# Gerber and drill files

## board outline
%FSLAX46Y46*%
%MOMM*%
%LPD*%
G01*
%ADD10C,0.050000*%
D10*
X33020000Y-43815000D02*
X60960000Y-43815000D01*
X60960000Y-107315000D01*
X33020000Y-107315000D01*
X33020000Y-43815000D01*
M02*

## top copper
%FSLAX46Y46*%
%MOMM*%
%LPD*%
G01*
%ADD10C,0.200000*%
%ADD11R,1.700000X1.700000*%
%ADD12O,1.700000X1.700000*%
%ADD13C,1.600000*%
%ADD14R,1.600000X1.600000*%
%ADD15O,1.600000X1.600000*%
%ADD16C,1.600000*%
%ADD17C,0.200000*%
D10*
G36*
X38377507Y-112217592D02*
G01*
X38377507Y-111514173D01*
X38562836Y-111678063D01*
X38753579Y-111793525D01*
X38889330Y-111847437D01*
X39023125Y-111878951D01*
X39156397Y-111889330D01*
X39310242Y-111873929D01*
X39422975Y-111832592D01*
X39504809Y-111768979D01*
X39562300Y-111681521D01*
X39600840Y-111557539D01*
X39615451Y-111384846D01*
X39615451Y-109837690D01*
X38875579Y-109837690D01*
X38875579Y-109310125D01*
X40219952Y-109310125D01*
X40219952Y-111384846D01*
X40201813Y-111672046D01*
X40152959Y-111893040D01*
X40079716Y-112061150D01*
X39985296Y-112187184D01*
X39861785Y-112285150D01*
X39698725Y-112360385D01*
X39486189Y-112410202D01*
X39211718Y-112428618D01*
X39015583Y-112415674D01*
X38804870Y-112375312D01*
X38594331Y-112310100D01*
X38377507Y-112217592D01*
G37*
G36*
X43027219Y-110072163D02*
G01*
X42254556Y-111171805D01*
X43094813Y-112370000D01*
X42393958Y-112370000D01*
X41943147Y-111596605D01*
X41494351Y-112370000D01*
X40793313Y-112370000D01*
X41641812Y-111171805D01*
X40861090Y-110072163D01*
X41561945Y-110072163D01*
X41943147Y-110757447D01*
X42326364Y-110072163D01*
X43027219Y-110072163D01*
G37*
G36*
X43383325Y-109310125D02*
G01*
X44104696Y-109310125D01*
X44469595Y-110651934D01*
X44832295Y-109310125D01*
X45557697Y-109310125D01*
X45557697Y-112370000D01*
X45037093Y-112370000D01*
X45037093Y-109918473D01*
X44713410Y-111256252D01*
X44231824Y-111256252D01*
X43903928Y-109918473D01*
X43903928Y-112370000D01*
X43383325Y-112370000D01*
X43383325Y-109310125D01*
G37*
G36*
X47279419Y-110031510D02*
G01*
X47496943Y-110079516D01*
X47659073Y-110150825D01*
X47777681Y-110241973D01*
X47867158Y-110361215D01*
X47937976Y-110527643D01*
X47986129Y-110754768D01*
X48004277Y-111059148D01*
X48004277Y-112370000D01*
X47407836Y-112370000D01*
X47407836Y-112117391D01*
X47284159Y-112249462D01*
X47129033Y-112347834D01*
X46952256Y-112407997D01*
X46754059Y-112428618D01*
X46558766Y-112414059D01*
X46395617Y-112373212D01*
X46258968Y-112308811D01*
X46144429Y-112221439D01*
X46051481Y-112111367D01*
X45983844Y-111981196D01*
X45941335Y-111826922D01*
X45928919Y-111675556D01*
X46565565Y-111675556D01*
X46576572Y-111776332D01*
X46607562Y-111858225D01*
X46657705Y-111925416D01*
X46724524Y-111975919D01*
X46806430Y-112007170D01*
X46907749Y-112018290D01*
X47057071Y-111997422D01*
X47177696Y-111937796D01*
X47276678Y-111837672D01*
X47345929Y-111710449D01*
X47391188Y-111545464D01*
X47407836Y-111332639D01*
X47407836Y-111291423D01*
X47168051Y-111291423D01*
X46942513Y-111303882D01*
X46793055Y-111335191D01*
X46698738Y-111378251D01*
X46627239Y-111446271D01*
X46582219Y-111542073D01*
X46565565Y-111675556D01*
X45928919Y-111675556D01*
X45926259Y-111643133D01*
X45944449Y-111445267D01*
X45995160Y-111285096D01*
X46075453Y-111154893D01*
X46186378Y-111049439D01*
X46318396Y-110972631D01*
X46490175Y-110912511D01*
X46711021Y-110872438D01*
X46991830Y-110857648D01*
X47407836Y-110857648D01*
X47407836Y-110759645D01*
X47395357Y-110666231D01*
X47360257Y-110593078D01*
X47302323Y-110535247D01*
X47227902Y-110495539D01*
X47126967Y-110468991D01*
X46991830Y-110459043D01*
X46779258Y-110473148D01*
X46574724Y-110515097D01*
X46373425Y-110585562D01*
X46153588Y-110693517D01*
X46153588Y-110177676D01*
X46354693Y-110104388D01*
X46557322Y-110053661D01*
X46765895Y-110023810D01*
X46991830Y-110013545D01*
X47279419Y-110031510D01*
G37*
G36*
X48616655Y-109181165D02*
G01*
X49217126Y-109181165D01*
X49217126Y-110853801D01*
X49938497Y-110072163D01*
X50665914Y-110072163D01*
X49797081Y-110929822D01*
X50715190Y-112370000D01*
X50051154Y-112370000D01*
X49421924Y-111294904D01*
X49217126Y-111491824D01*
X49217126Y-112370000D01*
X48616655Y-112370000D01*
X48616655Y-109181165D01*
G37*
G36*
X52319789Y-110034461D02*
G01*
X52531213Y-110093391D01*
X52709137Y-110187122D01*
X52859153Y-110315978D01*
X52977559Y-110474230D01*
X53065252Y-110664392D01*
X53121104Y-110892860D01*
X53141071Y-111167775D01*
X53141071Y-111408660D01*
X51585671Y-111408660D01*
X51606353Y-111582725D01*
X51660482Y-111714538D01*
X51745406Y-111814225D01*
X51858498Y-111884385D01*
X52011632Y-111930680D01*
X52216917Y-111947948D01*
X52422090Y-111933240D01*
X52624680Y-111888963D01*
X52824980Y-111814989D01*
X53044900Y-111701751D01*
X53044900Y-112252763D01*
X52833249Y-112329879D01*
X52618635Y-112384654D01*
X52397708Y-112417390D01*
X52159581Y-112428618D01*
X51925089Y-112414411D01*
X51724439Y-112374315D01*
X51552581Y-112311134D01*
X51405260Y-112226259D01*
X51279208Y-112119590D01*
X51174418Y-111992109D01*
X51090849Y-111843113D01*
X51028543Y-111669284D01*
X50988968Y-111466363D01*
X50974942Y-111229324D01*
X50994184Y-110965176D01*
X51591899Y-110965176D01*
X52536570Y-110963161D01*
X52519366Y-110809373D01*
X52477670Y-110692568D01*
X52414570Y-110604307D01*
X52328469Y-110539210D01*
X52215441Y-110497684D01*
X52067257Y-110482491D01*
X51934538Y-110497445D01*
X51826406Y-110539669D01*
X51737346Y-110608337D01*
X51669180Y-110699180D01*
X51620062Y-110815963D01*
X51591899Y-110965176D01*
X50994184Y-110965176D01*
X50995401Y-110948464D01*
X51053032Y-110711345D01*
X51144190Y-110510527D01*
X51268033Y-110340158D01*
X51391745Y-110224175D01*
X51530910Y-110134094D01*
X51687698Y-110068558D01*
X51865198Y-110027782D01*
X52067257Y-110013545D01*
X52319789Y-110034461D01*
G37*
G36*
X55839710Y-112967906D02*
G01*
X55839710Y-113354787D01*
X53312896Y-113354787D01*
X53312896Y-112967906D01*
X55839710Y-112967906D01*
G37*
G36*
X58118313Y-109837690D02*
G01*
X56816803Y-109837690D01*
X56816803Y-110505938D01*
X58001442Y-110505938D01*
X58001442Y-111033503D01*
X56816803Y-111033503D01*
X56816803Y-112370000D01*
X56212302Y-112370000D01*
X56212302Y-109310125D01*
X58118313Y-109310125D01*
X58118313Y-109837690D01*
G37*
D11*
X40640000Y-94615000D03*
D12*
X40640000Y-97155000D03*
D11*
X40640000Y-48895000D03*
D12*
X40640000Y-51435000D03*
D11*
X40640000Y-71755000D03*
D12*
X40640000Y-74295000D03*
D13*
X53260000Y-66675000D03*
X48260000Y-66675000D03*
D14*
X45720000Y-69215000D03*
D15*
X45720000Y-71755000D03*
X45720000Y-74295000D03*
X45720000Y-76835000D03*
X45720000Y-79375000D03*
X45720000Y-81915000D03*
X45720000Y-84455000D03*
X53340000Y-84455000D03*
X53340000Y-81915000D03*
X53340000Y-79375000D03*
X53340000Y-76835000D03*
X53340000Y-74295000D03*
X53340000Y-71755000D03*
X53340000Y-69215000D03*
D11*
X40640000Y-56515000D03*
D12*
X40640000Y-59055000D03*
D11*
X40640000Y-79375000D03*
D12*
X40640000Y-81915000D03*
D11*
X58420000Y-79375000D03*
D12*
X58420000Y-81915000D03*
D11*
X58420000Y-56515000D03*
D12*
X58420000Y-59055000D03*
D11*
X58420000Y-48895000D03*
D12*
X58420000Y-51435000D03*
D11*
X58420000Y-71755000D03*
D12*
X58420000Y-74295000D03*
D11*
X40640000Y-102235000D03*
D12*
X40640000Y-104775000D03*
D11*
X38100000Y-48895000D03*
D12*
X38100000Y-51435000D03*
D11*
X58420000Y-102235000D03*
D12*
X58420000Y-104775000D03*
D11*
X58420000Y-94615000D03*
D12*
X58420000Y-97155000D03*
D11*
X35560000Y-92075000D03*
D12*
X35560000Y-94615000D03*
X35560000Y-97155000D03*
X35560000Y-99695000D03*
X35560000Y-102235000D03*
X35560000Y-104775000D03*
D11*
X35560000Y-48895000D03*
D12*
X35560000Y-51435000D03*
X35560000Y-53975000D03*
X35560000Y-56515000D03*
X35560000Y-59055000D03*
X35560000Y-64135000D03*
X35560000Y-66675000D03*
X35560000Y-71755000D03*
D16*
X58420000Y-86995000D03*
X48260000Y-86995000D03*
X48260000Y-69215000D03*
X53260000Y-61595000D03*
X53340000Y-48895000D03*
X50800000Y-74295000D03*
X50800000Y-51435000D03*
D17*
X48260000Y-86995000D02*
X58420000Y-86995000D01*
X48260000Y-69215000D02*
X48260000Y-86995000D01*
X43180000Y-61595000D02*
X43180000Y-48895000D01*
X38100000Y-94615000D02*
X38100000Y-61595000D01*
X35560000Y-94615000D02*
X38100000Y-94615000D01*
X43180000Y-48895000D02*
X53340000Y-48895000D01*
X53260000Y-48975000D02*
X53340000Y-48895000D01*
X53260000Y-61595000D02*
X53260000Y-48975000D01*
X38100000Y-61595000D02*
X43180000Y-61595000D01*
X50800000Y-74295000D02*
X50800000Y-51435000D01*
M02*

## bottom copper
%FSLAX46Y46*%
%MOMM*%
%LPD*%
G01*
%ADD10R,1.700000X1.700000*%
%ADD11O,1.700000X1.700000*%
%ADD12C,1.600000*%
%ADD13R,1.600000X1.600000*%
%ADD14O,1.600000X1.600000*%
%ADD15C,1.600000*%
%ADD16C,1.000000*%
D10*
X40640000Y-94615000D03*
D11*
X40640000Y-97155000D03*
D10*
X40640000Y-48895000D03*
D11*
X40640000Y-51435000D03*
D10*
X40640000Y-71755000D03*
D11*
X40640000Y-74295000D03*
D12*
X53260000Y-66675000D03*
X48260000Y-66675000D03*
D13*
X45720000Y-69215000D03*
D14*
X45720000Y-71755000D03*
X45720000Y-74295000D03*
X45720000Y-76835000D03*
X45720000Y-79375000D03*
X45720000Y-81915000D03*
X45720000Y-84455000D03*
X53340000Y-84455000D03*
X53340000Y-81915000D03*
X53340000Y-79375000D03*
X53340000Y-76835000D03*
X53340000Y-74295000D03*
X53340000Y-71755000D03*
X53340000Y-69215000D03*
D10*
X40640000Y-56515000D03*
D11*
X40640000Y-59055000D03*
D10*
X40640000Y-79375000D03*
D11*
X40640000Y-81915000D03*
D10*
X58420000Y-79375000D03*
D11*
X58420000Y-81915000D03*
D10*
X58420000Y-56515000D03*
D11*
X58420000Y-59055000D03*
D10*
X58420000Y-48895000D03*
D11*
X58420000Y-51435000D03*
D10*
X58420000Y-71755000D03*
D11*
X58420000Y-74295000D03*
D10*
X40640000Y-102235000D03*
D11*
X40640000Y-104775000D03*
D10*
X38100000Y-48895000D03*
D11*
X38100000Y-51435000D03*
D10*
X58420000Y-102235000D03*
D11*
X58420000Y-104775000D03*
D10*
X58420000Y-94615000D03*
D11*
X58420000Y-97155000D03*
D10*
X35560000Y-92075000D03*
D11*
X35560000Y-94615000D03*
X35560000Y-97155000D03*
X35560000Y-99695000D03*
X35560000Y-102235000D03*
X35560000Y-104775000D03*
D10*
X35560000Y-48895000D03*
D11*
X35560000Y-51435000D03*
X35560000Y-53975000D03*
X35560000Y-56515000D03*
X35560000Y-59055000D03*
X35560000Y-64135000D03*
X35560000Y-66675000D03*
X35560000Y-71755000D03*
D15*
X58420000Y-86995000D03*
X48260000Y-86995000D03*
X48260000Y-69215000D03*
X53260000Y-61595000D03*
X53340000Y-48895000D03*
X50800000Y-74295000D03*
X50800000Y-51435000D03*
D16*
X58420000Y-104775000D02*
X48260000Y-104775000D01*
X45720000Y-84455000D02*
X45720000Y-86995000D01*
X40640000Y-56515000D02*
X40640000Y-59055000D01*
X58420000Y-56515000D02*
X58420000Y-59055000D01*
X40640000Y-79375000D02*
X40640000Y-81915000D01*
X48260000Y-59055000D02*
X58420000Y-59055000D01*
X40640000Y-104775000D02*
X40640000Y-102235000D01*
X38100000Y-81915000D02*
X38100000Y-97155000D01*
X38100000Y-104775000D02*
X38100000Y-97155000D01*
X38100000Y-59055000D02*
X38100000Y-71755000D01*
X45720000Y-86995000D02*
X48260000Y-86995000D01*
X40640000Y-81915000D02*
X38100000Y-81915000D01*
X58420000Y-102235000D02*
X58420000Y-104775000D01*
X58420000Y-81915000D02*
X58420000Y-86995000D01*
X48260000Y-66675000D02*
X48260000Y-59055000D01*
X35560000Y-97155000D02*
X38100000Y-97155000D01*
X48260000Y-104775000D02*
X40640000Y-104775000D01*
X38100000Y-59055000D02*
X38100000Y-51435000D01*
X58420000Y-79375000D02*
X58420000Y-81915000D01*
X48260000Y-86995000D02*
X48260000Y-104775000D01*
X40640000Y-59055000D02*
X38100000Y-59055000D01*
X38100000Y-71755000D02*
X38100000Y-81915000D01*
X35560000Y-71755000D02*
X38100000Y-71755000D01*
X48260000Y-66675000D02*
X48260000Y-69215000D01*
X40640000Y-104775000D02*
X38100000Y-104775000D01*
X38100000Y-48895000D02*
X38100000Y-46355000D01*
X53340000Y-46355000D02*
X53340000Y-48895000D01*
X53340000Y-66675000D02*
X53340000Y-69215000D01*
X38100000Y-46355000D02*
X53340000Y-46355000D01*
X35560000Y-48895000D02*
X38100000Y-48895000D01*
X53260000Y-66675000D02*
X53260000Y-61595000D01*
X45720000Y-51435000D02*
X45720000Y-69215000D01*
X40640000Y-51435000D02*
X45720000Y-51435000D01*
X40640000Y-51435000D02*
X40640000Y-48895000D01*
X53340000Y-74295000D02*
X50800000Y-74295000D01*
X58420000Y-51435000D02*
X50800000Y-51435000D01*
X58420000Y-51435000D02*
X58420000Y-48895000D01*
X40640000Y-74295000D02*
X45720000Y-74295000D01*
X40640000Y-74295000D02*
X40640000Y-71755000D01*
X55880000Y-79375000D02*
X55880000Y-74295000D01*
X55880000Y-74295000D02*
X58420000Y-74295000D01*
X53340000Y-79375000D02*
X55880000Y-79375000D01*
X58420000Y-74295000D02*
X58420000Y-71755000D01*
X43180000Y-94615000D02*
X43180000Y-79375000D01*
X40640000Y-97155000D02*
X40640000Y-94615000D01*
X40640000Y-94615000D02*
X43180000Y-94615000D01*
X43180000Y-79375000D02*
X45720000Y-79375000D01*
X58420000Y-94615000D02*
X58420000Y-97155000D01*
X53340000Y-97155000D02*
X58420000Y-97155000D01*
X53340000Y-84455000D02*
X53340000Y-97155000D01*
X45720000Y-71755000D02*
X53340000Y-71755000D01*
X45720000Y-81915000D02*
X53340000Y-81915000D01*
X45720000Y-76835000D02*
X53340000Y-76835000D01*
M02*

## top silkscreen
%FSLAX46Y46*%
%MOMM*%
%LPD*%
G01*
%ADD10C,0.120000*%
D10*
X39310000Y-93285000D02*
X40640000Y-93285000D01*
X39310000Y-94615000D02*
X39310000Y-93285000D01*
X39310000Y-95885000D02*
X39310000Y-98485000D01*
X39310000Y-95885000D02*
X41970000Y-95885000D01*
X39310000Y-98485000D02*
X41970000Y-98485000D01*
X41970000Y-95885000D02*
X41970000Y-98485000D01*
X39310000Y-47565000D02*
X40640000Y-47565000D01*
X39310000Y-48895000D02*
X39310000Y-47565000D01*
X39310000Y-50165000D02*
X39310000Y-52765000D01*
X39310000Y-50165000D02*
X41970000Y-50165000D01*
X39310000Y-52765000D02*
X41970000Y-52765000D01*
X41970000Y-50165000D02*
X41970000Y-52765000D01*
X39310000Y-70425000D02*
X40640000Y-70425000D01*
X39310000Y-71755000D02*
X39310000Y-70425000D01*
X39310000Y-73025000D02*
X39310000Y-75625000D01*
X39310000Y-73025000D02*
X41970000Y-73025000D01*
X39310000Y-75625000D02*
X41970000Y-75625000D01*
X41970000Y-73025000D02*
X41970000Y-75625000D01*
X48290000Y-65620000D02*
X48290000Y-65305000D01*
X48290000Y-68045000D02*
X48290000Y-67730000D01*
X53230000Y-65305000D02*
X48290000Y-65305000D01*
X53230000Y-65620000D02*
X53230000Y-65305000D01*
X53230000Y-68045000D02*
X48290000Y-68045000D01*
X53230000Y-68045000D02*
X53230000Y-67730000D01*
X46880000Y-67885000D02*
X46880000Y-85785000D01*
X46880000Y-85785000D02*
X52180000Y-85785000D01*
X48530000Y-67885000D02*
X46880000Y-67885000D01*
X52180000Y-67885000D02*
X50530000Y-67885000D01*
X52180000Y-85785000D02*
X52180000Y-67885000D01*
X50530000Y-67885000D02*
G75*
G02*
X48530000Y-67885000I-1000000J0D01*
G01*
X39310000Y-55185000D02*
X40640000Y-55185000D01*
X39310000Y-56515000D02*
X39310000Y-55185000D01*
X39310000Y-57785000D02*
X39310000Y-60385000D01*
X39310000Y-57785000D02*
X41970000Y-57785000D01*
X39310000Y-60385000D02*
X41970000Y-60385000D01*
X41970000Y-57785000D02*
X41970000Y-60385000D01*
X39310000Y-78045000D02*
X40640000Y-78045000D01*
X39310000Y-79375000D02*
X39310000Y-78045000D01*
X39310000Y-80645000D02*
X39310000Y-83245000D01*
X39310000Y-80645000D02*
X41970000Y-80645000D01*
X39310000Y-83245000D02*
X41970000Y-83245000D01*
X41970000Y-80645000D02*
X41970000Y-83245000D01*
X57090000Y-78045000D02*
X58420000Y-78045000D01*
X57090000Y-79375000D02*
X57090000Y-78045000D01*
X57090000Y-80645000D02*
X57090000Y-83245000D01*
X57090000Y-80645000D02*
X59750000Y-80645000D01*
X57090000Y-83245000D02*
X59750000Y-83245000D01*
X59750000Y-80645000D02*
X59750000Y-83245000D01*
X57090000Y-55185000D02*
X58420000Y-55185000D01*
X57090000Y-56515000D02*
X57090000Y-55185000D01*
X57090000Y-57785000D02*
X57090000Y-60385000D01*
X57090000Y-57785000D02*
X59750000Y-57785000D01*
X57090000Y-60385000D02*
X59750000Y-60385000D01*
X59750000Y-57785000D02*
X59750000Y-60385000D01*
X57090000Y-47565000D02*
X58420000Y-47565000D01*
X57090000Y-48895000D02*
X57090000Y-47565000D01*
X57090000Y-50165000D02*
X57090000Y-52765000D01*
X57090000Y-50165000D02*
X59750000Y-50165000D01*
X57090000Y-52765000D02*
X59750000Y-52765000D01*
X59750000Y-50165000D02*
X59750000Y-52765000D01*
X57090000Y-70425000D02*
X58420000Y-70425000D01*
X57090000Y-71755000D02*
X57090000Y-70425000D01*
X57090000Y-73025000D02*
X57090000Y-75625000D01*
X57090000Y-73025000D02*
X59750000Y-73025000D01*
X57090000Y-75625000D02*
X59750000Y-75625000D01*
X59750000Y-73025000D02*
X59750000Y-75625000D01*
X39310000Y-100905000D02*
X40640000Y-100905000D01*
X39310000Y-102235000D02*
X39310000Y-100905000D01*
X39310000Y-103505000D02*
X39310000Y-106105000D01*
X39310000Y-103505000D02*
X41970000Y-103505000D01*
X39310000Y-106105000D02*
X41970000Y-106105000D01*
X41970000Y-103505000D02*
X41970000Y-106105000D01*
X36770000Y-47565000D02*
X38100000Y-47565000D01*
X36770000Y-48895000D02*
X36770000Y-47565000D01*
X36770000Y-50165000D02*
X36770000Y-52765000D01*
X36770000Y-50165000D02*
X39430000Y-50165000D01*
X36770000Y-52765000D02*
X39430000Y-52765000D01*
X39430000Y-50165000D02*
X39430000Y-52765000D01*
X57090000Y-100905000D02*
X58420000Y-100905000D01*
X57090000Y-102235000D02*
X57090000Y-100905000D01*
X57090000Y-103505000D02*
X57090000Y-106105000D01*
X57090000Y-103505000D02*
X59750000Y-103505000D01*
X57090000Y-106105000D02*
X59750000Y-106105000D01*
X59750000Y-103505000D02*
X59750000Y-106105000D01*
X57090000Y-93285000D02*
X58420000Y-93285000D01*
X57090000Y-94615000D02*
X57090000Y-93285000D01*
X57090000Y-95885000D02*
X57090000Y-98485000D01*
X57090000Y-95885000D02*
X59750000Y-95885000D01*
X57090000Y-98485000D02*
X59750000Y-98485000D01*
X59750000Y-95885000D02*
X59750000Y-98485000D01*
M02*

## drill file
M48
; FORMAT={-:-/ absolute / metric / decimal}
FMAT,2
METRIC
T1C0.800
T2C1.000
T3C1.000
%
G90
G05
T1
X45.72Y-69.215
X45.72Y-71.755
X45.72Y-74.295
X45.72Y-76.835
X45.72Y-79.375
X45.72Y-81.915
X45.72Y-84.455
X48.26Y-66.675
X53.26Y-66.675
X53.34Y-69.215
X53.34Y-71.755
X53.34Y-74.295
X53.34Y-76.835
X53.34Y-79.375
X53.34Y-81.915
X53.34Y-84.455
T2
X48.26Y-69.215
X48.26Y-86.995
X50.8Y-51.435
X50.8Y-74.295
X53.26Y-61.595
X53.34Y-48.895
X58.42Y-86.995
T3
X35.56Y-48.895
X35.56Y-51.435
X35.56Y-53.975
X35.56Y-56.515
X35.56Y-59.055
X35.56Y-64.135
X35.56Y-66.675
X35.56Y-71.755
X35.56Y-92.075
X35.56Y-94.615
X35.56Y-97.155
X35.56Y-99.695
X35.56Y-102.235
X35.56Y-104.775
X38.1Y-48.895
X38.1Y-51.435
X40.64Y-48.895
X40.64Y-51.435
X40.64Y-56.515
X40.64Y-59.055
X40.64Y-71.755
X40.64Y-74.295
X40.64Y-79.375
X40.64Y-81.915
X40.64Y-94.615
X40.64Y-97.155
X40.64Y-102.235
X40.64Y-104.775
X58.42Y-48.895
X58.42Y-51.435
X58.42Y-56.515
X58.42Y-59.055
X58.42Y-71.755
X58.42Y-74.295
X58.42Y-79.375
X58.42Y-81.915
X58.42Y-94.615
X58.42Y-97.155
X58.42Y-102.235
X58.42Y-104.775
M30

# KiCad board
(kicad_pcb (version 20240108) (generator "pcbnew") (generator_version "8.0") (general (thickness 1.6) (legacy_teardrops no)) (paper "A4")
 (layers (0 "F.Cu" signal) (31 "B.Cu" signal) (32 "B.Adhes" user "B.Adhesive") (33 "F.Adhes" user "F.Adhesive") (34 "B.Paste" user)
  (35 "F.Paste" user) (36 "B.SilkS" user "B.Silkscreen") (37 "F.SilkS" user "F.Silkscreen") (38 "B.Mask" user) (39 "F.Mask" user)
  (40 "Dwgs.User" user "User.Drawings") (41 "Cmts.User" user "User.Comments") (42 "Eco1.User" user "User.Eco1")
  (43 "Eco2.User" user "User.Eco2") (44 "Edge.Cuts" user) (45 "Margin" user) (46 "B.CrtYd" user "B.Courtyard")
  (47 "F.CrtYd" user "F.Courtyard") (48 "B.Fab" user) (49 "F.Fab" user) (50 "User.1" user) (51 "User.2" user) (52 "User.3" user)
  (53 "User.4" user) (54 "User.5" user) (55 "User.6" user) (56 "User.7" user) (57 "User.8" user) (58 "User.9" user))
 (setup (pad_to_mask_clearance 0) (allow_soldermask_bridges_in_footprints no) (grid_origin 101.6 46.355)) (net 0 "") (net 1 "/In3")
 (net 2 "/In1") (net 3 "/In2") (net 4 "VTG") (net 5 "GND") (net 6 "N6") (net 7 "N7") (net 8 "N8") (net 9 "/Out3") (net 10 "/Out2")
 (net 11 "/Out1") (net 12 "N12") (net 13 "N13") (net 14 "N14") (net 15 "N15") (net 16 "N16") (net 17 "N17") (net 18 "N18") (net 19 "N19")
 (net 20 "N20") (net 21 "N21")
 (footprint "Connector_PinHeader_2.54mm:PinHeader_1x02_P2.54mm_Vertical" (layer "F.Cu") (at 40.64 94.615)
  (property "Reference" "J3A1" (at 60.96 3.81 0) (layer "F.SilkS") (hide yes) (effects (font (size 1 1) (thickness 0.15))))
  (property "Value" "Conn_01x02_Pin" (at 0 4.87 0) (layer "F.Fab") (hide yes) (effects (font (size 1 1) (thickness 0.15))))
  (fp_line (start -1.33 -1.33) (end 0 -1.33) (stroke (width 0.12) (type solid)) (layer "F.SilkS"))
  (fp_line (start -1.33 0) (end -1.33 -1.33) (stroke (width 0.12) (type solid)) (layer "F.SilkS"))
  (fp_line (start -1.33 1.27) (end -1.33 3.87) (stroke (width 0.12) (type solid)) (layer "F.SilkS"))
  (fp_line (start -1.33 1.27) (end 1.33 1.27) (stroke (width 0.12) (type solid)) (layer "F.SilkS"))
  (fp_line (start -1.33 3.87) (end 1.33 3.87) (stroke (width 0.12) (type solid)) (layer "F.SilkS"))
  (fp_line (start 1.33 1.27) (end 1.33 3.87) (stroke (width 0.12) (type solid)) (layer "F.SilkS"))
  (pad "1" thru_hole rect (at 0 0) (size 1.7 1.7) (drill 1) (layers "*.Cu" "*.Mask") (remove_unused_layers no) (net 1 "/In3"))
  (pad "2" thru_hole oval (at 0 2.54) (size 1.7 1.7) (drill 1) (layers "*.Cu" "*.Mask") (remove_unused_layers no) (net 1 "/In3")))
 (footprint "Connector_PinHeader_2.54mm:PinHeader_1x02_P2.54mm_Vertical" (layer "F.Cu") (at 40.64 48.895)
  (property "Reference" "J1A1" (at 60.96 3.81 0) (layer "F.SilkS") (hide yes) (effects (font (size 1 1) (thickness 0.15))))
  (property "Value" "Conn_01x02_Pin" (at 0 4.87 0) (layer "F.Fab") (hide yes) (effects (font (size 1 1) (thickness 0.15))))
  (fp_line (start -1.33 -1.33) (end 0 -1.33) (stroke (width 0.12) (type solid)) (layer "F.SilkS"))
  (fp_line (start -1.33 0) (end -1.33 -1.33) (stroke (width 0.12) (type solid)) (layer "F.SilkS"))
  (fp_line (start -1.33 1.27) (end -1.33 3.87) (stroke (width 0.12) (type solid)) (layer "F.SilkS"))
  (fp_line (start -1.33 1.27) (end 1.33 1.27) (stroke (width 0.12) (type solid)) (layer "F.SilkS"))
  (fp_line (start -1.33 3.87) (end 1.33 3.87) (stroke (width 0.12) (type solid)) (layer "F.SilkS"))
  (fp_line (start 1.33 1.27) (end 1.33 3.87) (stroke (width 0.12) (type solid)) (layer "F.SilkS"))
  (pad "1" thru_hole rect (at 0 0) (size 1.7 1.7) (drill 1) (layers "*.Cu" "*.Mask") (remove_unused_layers no) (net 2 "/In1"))
  (pad "2" thru_hole oval (at 0 2.54) (size 1.7 1.7) (drill 1) (layers "*.Cu" "*.Mask") (remove_unused_layers no) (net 2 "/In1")))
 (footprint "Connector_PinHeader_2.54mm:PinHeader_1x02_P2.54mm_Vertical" (layer "F.Cu") (at 40.64 71.755)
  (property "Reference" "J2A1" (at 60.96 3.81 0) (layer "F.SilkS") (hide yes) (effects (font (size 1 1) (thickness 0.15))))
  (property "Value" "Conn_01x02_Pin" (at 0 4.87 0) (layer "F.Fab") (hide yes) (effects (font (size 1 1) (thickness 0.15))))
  (fp_line (start -1.33 -1.33) (end 0 -1.33) (stroke (width 0.12) (type solid)) (layer "F.SilkS"))
  (fp_line (start -1.33 0) (end -1.33 -1.33) (stroke (width 0.12) (type solid)) (layer "F.SilkS"))
  (fp_line (start -1.33 1.27) (end -1.33 3.87) (stroke (width 0.12) (type solid)) (layer "F.SilkS"))
  (fp_line (start -1.33 1.27) (end 1.33 1.27) (stroke (width 0.12) (type solid)) (layer "F.SilkS"))
  (fp_line (start -1.33 3.87) (end 1.33 3.87) (stroke (width 0.12) (type solid)) (layer "F.SilkS"))
  (fp_line (start 1.33 1.27) (end 1.33 3.87) (stroke (width 0.12) (type solid)) (layer "F.SilkS"))
  (pad "1" thru_hole rect (at 0 0) (size 1.7 1.7) (drill 1) (layers "*.Cu" "*.Mask") (remove_unused_layers no) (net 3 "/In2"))
  (pad "2" thru_hole oval (at 0 2.54) (size 1.7 1.7) (drill 1) (layers "*.Cu" "*.Mask") (remove_unused_layers no) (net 3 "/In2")))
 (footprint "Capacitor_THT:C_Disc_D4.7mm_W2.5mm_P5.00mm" (layer "F.Cu") (at 53.26 66.675 180)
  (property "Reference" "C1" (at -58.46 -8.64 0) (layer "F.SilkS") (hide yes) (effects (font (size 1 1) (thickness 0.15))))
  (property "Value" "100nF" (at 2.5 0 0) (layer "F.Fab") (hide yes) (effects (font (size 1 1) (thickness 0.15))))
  (fp_line (start 4.97 1.055) (end 4.97 1.37) (stroke (width 0.12) (type solid)) (layer "F.SilkS"))
  (fp_line (start 4.97 -1.37) (end 4.97 -1.055) (stroke (width 0.12) (type solid)) (layer "F.SilkS"))
  (fp_line (start 0.03 1.37) (end 4.97 1.37) (stroke (width 0.12) (type solid)) (layer "F.SilkS"))
  (fp_line (start 0.03 1.055) (end 0.03 1.37) (stroke (width 0.12) (type solid)) (layer "F.SilkS"))
  (fp_line (start 0.03 -1.37) (end 4.97 -1.37) (stroke (width 0.12) (type solid)) (layer "F.SilkS"))
  (fp_line (start 0.03 -1.37) (end 0.03 -1.055) (stroke (width 0.12) (type solid)) (layer "F.SilkS"))
  (pad "1" thru_hole circle (at 0 0 180) (size 1.6 1.6) (drill 0.8) (layers "*.Cu" "*.Mask") (remove_unused_layers no) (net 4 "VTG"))
  (pad "2" thru_hole circle (at 5 0 180) (size 1.6 1.6) (drill 0.8) (layers "*.Cu" "*.Mask") (remove_unused_layers no) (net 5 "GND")))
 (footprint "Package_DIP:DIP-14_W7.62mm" (layer "F.Cu") (at 45.72 69.215)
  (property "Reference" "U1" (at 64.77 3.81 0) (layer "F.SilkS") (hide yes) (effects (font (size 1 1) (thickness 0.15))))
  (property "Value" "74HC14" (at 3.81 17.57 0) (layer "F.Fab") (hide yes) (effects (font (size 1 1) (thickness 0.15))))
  (fp_line (start 1.16 -1.33) (end 1.16 16.57) (stroke (width 0.12) (type solid)) (layer "F.SilkS"))
  (fp_line (start 1.16 16.57) (end 6.46 16.57) (stroke (width 0.12) (type solid)) (layer "F.SilkS"))
  (fp_line (start 2.81 -1.33) (end 1.16 -1.33) (stroke (width 0.12) (type solid)) (layer "F.SilkS"))
  (fp_line (start 6.46 -1.33) (end 4.81 -1.33) (stroke (width 0.12) (type solid)) (layer "F.SilkS"))
  (fp_line (start 6.46 16.57) (end 6.46 -1.33) (stroke (width 0.12) (type solid)) (layer "F.SilkS"))
  (fp_arc (start 4.81 -1.33) (mid 3.81 -0.33) (end 2.81 -1.33) (stroke (width 0.12) (type solid)) (layer "F.SilkS"))
  (pad "1" thru_hole rect (at 0 0) (size 1.6 1.6) (drill 0.8) (layers "*.Cu" "*.Mask") (remove_unused_layers no) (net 2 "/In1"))
  (pad "2" thru_hole oval (at 0 2.54) (size 1.6 1.6) (drill 0.8) (layers "*.Cu" "*.Mask") (remove_unused_layers no) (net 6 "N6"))
  (pad "3" thru_hole oval (at 0 5.08) (size 1.6 1.6) (drill 0.8) (layers "*.Cu" "*.Mask") (remove_unused_layers no) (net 3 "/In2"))
  (pad "4" thru_hole oval (at 0 7.62) (size 1.6 1.6) (drill 0.8) (layers "*.Cu" "*.Mask") (remove_unused_layers no) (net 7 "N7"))
  (pad "5" thru_hole oval (at 0 10.16) (size 1.6 1.6) (drill 0.8) (layers "*.Cu" "*.Mask") (remove_unused_layers no) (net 1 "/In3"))
  (pad "6" thru_hole oval (at 0 12.7) (size 1.6 1.6) (drill 0.8) (layers "*.Cu" "*.Mask") (remove_unused_layers no) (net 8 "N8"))
  (pad "7" thru_hole oval (at 0 15.24) (size 1.6 1.6) (drill 0.8) (layers "*.Cu" "*.Mask") (remove_unused_layers no) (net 5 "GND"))
  (pad "8" thru_hole oval (at 7.62 15.24) (size 1.6 1.6) (drill 0.8) (layers "*.Cu" "*.Mask") (remove_unused_layers no) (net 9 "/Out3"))
  (pad "9" thru_hole oval (at 7.62 12.7) (size 1.6 1.6) (drill 0.8) (layers "*.Cu" "*.Mask") (remove_unused_layers no) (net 8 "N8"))
  (pad "10" thru_hole oval (at 7.62 10.16) (size 1.6 1.6) (drill 0.8) (layers "*.Cu" "*.Mask") (remove_unused_layers no) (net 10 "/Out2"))
  (pad "11" thru_hole oval (at 7.62 7.62) (size 1.6 1.6) (drill 0.8) (layers "*.Cu" "*.Mask") (remove_unused_layers no) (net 7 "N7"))
  (pad "12" thru_hole oval (at 7.62 5.08) (size 1.6 1.6) (drill 0.8) (layers "*.Cu" "*.Mask") (remove_unused_layers no) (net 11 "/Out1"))
  (pad "13" thru_hole oval (at 7.62 2.54) (size 1.6 1.6) (drill 0.8) (layers "*.Cu" "*.Mask") (remove_unused_layers no) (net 6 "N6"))
  (pad "14" thru_hole oval (at 7.62 0) (size 1.6 1.6) (drill 0.8) (layers "*.Cu" "*.Mask") (remove_unused_layers no) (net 4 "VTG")))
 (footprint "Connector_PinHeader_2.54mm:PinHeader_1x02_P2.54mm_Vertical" (layer "F.Cu") (at 40.64 56.515)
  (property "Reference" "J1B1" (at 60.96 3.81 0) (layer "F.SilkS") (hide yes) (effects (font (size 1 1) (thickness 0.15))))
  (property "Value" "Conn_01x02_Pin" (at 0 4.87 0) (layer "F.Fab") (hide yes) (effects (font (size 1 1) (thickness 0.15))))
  (fp_line (start -1.33 -1.33) (end 0 -1.33) (stroke (width 0.12) (type solid)) (layer "F.SilkS"))
  (fp_line (start -1.33 0) (end -1.33 -1.33) (stroke (width 0.12) (type solid)) (layer "F.SilkS"))
  (fp_line (start -1.33 1.27) (end -1.33 3.87) (stroke (width 0.12) (type solid)) (layer "F.SilkS"))
  (fp_line (start -1.33 1.27) (end 1.33 1.27) (stroke (width 0.12) (type solid)) (layer "F.SilkS"))
  (fp_line (start -1.33 3.87) (end 1.33 3.87) (stroke (width 0.12) (type solid)) (layer "F.SilkS"))
  (fp_line (start 1.33 1.27) (end 1.33 3.87) (stroke (width 0.12) (type solid)) (layer "F.SilkS"))
  (pad "1" thru_hole rect (at 0 0) (size 1.7 1.7) (drill 1) (layers "*.Cu" "*.Mask") (remove_unused_layers no) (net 5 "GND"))
  (pad "2" thru_hole oval (at 0 2.54) (size 1.7 1.7) (drill 1) (layers "*.Cu" "*.Mask") (remove_unused_layers no) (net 5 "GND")))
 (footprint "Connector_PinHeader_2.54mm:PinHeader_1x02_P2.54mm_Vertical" (layer "F.Cu") (at 40.64 79.375)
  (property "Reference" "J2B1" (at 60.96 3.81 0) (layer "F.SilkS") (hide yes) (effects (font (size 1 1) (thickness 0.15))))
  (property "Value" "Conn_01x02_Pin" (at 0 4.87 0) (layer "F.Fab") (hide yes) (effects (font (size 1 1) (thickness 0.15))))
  (fp_line (start -1.33 -1.33) (end 0 -1.33) (stroke (width 0.12) (type solid)) (layer "F.SilkS"))
  (fp_line (start -1.33 0) (end -1.33 -1.33) (stroke (width 0.12) (type solid)) (layer "F.SilkS"))
  (fp_line (start -1.33 1.27) (end -1.33 3.87) (stroke (width 0.12) (type solid)) (layer "F.SilkS"))
  (fp_line (start -1.33 1.27) (end 1.33 1.27) (stroke (width 0.12) (type solid)) (layer "F.SilkS"))
  (fp_line (start -1.33 3.87) (end 1.33 3.87) (stroke (width 0.12) (type solid)) (layer "F.SilkS"))
  (fp_line (start 1.33 1.27) (end 1.33 3.87) (stroke (width 0.12) (type solid)) (layer "F.SilkS"))
  (pad "1" thru_hole rect (at 0 0) (size 1.7 1.7) (drill 1) (layers "*.Cu" "*.Mask") (remove_unused_layers no) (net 5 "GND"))
  (pad "2" thru_hole oval (at 0 2.54) (size 1.7 1.7) (drill 1) (layers "*.Cu" "*.Mask") (remove_unused_layers no) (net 5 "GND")))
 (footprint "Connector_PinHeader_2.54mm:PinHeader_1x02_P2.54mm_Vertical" (layer "F.Cu") (at 58.42 79.375)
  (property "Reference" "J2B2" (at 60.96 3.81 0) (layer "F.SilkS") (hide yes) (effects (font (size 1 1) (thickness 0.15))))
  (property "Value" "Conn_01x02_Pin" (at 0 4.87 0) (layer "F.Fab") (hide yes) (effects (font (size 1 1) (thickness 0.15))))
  (fp_line (start -1.33 -1.33) (end 0 -1.33) (stroke (width 0.12) (type solid)) (layer "F.SilkS"))
  (fp_line (start -1.33 0) (end -1.33 -1.33) (stroke (width 0.12) (type solid)) (layer "F.SilkS"))
  (fp_line (start -1.33 1.27) (end -1.33 3.87) (stroke (width 0.12) (type solid)) (layer "F.SilkS"))
  (fp_line (start -1.33 1.27) (end 1.33 1.27) (stroke (width 0.12) (type solid)) (layer "F.SilkS"))
  (fp_line (start -1.33 3.87) (end 1.33 3.87) (stroke (width 0.12) (type solid)) (layer "F.SilkS"))
  (fp_line (start 1.33 1.27) (end 1.33 3.87) (stroke (width 0.12) (type solid)) (layer "F.SilkS"))
  (pad "1" thru_hole rect (at 0 0) (size 1.7 1.7) (drill 1) (layers "*.Cu" "*.Mask") (remove_unused_layers no) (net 5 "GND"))
  (pad "2" thru_hole oval (at 0 2.54) (size 1.7 1.7) (drill 1) (layers "*.Cu" "*.Mask") (remove_unused_layers no) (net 5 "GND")))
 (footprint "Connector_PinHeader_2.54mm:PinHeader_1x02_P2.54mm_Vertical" (layer "F.Cu") (at 58.42 56.515)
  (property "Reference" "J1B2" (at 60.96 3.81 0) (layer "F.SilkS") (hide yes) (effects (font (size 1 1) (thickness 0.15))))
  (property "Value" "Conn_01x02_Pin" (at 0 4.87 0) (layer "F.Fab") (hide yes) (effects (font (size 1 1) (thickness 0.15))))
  (fp_line (start -1.33 -1.33) (end 0 -1.33) (stroke (width 0.12) (type solid)) (layer "F.SilkS"))
  (fp_line (start -1.33 0) (end -1.33 -1.33) (stroke (width 0.12) (type solid)) (layer "F.SilkS"))
  (fp_line (start -1.33 1.27) (end -1.33 3.87) (stroke (width 0.12) (type solid)) (layer "F.SilkS"))
  (fp_line (start -1.33 1.27) (end 1.33 1.27) (stroke (width 0.12) (type solid)) (layer "F.SilkS"))
  (fp_line (start -1.33 3.87) (end 1.33 3.87) (stroke (width 0.12) (type solid)) (layer "F.SilkS"))
  (fp_line (start 1.33 1.27) (end 1.33 3.87) (stroke (width 0.12) (type solid)) (layer "F.SilkS"))
  (pad "1" thru_hole rect (at 0 0) (size 1.7 1.7) (drill 1) (layers "*.Cu" "*.Mask") (remove_unused_layers no) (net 5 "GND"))
  (pad "2" thru_hole oval (at 0 2.54) (size 1.7 1.7) (drill 1) (layers "*.Cu" "*.Mask") (remove_unused_layers no) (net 5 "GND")))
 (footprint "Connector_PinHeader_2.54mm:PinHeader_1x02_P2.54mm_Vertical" (layer "F.Cu") (at 58.42 48.895)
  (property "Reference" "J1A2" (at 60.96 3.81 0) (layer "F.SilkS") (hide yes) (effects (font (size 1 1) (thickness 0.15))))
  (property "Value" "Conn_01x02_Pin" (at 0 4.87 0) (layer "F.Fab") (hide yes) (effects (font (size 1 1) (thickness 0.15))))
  (fp_line (start -1.33 -1.33) (end 0 -1.33) (stroke (width 0.12) (type solid)) (layer "F.SilkS"))
  (fp_line (start -1.33 0) (end -1.33 -1.33) (stroke (width 0.12) (type solid)) (layer "F.SilkS"))
  (fp_line (start -1.33 1.27) (end -1.33 3.87) (stroke (width 0.12) (type solid)) (layer "F.SilkS"))
  (fp_line (start -1.33 1.27) (end 1.33 1.27) (stroke (width 0.12) (type solid)) (layer "F.SilkS"))
  (fp_line (start -1.33 3.87) (end 1.33 3.87) (stroke (width 0.12) (type solid)) (layer "F.SilkS"))
  (fp_line (start 1.33 1.27) (end 1.33 3.87) (stroke (width 0.12) (type solid)) (layer "F.SilkS"))
  (pad "1" thru_hole rect (at 0 0) (size 1.7 1.7) (drill 1) (layers "*.Cu" "*.Mask") (remove_unused_layers no) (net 11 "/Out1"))
  (pad "2" thru_hole oval (at 0 2.54) (size 1.7 1.7) (drill 1) (layers "*.Cu" "*.Mask") (remove_unused_layers no) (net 11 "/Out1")))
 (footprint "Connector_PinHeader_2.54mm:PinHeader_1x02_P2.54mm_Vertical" (layer "F.Cu") (at 58.42 71.755)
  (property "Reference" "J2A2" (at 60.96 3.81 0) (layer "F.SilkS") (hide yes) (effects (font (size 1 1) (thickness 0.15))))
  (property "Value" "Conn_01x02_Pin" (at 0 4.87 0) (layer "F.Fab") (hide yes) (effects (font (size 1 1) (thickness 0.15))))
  (fp_line (start -1.33 -1.33) (end 0 -1.33) (stroke (width 0.12) (type solid)) (layer "F.SilkS"))
  (fp_line (start -1.33 0) (end -1.33 -1.33) (stroke (width 0.12) (type solid)) (layer "F.SilkS"))
  (fp_line (start -1.33 1.27) (end -1.33 3.87) (stroke (width 0.12) (type solid)) (layer "F.SilkS"))
  (fp_line (start -1.33 1.27) (end 1.33 1.27) (stroke (width 0.12) (type solid)) (layer "F.SilkS"))
  (fp_line (start -1.33 3.87) (end 1.33 3.87) (stroke (width 0.12) (type solid)) (layer "F.SilkS"))
  (fp_line (start 1.33 1.27) (end 1.33 3.87) (stroke (width 0.12) (type solid)) (layer "F.SilkS"))
  (pad "1" thru_hole rect (at 0 0) (size 1.7 1.7) (drill 1) (layers "*.Cu" "*.Mask") (remove_unused_layers no) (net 10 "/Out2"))
  (pad "2" thru_hole oval (at 0 2.54) (size 1.7 1.7) (drill 1) (layers "*.Cu" "*.Mask") (remove_unused_layers no) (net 10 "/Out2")))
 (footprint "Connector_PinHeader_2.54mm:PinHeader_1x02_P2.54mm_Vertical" (layer "F.Cu") (at 40.64 102.235)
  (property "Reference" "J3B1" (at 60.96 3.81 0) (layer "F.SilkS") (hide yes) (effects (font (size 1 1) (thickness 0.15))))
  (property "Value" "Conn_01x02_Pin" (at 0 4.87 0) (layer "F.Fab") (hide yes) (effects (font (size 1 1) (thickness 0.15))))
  (fp_line (start -1.33 -1.33) (end 0 -1.33) (stroke (width 0.12) (type solid)) (layer "F.SilkS"))
  (fp_line (start -1.33 0) (end -1.33 -1.33) (stroke (width 0.12) (type solid)) (layer "F.SilkS"))
  (fp_line (start -1.33 1.27) (end -1.33 3.87) (stroke (width 0.12) (type solid)) (layer "F.SilkS"))
  (fp_line (start -1.33 1.27) (end 1.33 1.27) (stroke (width 0.12) (type solid)) (layer "F.SilkS"))
  (fp_line (start -1.33 3.87) (end 1.33 3.87) (stroke (width 0.12) (type solid)) (layer "F.SilkS"))
  (fp_line (start 1.33 1.27) (end 1.33 3.87) (stroke (width 0.12) (type solid)) (layer "F.SilkS"))
  (pad "1" thru_hole rect (at 0 0) (size 1.7 1.7) (drill 1) (layers "*.Cu" "*.Mask") (remove_unused_layers no) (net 5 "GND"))
  (pad "2" thru_hole oval (at 0 2.54) (size 1.7 1.7) (drill 1) (layers "*.Cu" "*.Mask") (remove_unused_layers no) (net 5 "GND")))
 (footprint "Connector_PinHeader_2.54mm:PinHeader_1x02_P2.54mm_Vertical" (layer "F.Cu") (at 38.1 48.895)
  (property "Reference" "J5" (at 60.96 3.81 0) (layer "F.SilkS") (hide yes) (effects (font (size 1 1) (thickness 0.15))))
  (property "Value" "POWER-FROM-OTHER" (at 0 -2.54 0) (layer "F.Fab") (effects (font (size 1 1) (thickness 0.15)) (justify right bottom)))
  (fp_line (start -1.33 -1.33) (end 0 -1.33) (stroke (width 0.12) (type solid)) (layer "F.SilkS"))
  (fp_line (start -1.33 0) (end -1.33 -1.33) (stroke (width 0.12) (type solid)) (layer "F.SilkS"))
  (fp_line (start -1.33 1.27) (end -1.33 3.87) (stroke (width 0.12) (type solid)) (layer "F.SilkS"))
  (fp_line (start -1.33 1.27) (end 1.33 1.27) (stroke (width 0.12) (type solid)) (layer "F.SilkS"))
  (fp_line (start -1.33 3.87) (end 1.33 3.87) (stroke (width 0.12) (type solid)) (layer "F.SilkS"))
  (fp_line (start 1.33 1.27) (end 1.33 3.87) (stroke (width 0.12) (type solid)) (layer "F.SilkS"))
  (pad "1" thru_hole rect (at 0 0) (size 1.7 1.7) (drill 1) (layers "*.Cu" "*.Mask") (remove_unused_layers no) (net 4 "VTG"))
  (pad "2" thru_hole oval (at 0 2.54) (size 1.7 1.7) (drill 1) (layers "*.Cu" "*.Mask") (remove_unused_layers no) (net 5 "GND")))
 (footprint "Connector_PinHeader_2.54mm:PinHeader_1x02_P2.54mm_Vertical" (layer "F.Cu") (at 58.42 102.235)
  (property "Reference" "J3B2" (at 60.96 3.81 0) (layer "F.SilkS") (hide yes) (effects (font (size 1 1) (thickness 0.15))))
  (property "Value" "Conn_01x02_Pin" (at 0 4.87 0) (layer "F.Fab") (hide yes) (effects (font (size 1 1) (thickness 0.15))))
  (fp_line (start -1.33 -1.33) (end 0 -1.33) (stroke (width 0.12) (type solid)) (layer "F.SilkS"))
  (fp_line (start -1.33 0) (end -1.33 -1.33) (stroke (width 0.12) (type solid)) (layer "F.SilkS"))
  (fp_line (start -1.33 1.27) (end -1.33 3.87) (stroke (width 0.12) (type solid)) (layer "F.SilkS"))
  (fp_line (start -1.33 1.27) (end 1.33 1.27) (stroke (width 0.12) (type solid)) (layer "F.SilkS"))
  (fp_line (start -1.33 3.87) (end 1.33 3.87) (stroke (width 0.12) (type solid)) (layer "F.SilkS"))
  (fp_line (start 1.33 1.27) (end 1.33 3.87) (stroke (width 0.12) (type solid)) (layer "F.SilkS"))
  (pad "1" thru_hole rect (at 0 0) (size 1.7 1.7) (drill 1) (layers "*.Cu" "*.Mask") (remove_unused_layers no) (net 5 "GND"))
  (pad "2" thru_hole oval (at 0 2.54) (size 1.7 1.7) (drill 1) (layers "*.Cu" "*.Mask") (remove_unused_layers no) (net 5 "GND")))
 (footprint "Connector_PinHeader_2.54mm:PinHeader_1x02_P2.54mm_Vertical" (layer "F.Cu") (at 58.42 94.615)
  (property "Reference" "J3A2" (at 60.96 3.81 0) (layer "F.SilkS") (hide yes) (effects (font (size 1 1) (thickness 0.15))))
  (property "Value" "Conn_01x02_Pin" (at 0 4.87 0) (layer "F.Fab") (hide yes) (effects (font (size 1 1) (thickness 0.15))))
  (fp_line (start -1.33 -1.33) (end 0 -1.33) (stroke (width 0.12) (type solid)) (layer "F.SilkS"))
  (fp_line (start -1.33 0) (end -1.33 -1.33) (stroke (width 0.12) (type solid)) (layer "F.SilkS"))
  (fp_line (start -1.33 1.27) (end -1.33 3.87) (stroke (width 0.12) (type solid)) (layer "F.SilkS"))
  (fp_line (start -1.33 1.27) (end 1.33 1.27) (stroke (width 0.12) (type solid)) (layer "F.SilkS"))
  (fp_line (start -1.33 3.87) (end 1.33 3.87) (stroke (width 0.12) (type solid)) (layer "F.SilkS"))
  (fp_line (start 1.33 1.27) (end 1.33 3.87) (stroke (width 0.12) (type solid)) (layer "F.SilkS"))
  (pad "1" thru_hole rect (at 0 0) (size 1.7 1.7) (drill 1) (layers "*.Cu" "*.Mask") (remove_unused_layers no) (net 9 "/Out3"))
  (pad "2" thru_hole oval (at 0 2.54) (size 1.7 1.7) (drill 1) (layers "*.Cu" "*.Mask") (remove_unused_layers no) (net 9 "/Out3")))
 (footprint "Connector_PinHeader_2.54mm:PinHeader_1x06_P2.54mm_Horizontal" (layer "B.Cu") (at 35.56 92.075 180)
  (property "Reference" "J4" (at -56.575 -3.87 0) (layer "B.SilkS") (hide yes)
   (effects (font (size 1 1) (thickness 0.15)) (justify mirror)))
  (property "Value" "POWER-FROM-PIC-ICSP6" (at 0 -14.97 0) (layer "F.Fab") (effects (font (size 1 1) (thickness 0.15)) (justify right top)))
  (pad "1" thru_hole rect (at 0 0 180) (size 1.7 1.7) (drill 1) (layers "*.Cu" "*.Mask") (remove_unused_layers no) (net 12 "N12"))
  (pad "2" thru_hole oval (at 0 -2.54 180) (size 1.7 1.7) (drill 1) (layers "*.Cu" "*.Mask") (remove_unused_layers no) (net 4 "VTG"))
  (pad "3" thru_hole oval (at 0 -5.08 180) (size 1.7 1.7) (drill 1) (layers "*.Cu" "*.Mask") (remove_unused_layers no) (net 5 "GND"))
  (pad "4" thru_hole oval (at 0 -7.62 180) (size 1.7 1.7) (drill 1) (layers "*.Cu" "*.Mask") (remove_unused_layers no) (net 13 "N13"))
  (pad "5" thru_hole oval (at 0 -10.16 180) (size 1.7 1.7) (drill 1) (layers "*.Cu" "*.Mask") (remove_unused_layers no) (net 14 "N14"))
  (pad "6" thru_hole oval (at 0 -12.7 180) (size 1.7 1.7) (drill 1) (layers "*.Cu" "*.Mask") (remove_unused_layers no) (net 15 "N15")))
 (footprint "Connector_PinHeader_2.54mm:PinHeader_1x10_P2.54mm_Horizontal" (layer "B.Cu") (at 35.56 48.895 180)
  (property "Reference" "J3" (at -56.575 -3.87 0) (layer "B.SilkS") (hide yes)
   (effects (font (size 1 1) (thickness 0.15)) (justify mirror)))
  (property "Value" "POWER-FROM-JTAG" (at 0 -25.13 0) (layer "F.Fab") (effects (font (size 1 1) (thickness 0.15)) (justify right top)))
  (pad "1" thru_hole rect (at 0 0 180) (size 1.7 1.7) (drill 1) (layers "*.Cu" "*.Mask") (remove_unused_layers no) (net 4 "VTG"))
  (pad "2" thru_hole oval (at 0 -2.54 180) (size 1.7 1.7) (drill 1) (layers "*.Cu" "*.Mask") (remove_unused_layers no) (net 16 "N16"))
  (pad "3" thru_hole oval (at 0 -5.08 180) (size 1.7 1.7) (drill 1) (layers "*.Cu" "*.Mask") (remove_unused_layers no) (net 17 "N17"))
  (pad "4" thru_hole oval (at 0 -7.62 180) (size 1.7 1.7) (drill 1) (layers "*.Cu" "*.Mask") (remove_unused_layers no) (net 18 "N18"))
  (pad "5" thru_hole oval (at 0 -10.16 180) (size 1.7 1.7) (drill 1) (layers "*.Cu" "*.Mask") (remove_unused_layers no) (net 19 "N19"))
  (pad "7" thru_hole oval (at 0 -15.24 180) (size 1.7 1.7) (drill 1) (layers "*.Cu" "*.Mask") (remove_unused_layers no) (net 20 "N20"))
  (pad "8" thru_hole oval (at 0 -17.78 180) (size 1.7 1.7) (drill 1) (layers "*.Cu" "*.Mask") (remove_unused_layers no) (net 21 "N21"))
  (pad "10" thru_hole oval (at 0 -22.86 180) (size 1.7 1.7) (drill 1) (layers "*.Cu" "*.Mask") (remove_unused_layers no) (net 5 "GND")))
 (gr_rect (start 33.02 43.815) (end 60.96 107.315) (stroke (width 0.05) (type default)) (fill none) (layer "Edge.Cuts"))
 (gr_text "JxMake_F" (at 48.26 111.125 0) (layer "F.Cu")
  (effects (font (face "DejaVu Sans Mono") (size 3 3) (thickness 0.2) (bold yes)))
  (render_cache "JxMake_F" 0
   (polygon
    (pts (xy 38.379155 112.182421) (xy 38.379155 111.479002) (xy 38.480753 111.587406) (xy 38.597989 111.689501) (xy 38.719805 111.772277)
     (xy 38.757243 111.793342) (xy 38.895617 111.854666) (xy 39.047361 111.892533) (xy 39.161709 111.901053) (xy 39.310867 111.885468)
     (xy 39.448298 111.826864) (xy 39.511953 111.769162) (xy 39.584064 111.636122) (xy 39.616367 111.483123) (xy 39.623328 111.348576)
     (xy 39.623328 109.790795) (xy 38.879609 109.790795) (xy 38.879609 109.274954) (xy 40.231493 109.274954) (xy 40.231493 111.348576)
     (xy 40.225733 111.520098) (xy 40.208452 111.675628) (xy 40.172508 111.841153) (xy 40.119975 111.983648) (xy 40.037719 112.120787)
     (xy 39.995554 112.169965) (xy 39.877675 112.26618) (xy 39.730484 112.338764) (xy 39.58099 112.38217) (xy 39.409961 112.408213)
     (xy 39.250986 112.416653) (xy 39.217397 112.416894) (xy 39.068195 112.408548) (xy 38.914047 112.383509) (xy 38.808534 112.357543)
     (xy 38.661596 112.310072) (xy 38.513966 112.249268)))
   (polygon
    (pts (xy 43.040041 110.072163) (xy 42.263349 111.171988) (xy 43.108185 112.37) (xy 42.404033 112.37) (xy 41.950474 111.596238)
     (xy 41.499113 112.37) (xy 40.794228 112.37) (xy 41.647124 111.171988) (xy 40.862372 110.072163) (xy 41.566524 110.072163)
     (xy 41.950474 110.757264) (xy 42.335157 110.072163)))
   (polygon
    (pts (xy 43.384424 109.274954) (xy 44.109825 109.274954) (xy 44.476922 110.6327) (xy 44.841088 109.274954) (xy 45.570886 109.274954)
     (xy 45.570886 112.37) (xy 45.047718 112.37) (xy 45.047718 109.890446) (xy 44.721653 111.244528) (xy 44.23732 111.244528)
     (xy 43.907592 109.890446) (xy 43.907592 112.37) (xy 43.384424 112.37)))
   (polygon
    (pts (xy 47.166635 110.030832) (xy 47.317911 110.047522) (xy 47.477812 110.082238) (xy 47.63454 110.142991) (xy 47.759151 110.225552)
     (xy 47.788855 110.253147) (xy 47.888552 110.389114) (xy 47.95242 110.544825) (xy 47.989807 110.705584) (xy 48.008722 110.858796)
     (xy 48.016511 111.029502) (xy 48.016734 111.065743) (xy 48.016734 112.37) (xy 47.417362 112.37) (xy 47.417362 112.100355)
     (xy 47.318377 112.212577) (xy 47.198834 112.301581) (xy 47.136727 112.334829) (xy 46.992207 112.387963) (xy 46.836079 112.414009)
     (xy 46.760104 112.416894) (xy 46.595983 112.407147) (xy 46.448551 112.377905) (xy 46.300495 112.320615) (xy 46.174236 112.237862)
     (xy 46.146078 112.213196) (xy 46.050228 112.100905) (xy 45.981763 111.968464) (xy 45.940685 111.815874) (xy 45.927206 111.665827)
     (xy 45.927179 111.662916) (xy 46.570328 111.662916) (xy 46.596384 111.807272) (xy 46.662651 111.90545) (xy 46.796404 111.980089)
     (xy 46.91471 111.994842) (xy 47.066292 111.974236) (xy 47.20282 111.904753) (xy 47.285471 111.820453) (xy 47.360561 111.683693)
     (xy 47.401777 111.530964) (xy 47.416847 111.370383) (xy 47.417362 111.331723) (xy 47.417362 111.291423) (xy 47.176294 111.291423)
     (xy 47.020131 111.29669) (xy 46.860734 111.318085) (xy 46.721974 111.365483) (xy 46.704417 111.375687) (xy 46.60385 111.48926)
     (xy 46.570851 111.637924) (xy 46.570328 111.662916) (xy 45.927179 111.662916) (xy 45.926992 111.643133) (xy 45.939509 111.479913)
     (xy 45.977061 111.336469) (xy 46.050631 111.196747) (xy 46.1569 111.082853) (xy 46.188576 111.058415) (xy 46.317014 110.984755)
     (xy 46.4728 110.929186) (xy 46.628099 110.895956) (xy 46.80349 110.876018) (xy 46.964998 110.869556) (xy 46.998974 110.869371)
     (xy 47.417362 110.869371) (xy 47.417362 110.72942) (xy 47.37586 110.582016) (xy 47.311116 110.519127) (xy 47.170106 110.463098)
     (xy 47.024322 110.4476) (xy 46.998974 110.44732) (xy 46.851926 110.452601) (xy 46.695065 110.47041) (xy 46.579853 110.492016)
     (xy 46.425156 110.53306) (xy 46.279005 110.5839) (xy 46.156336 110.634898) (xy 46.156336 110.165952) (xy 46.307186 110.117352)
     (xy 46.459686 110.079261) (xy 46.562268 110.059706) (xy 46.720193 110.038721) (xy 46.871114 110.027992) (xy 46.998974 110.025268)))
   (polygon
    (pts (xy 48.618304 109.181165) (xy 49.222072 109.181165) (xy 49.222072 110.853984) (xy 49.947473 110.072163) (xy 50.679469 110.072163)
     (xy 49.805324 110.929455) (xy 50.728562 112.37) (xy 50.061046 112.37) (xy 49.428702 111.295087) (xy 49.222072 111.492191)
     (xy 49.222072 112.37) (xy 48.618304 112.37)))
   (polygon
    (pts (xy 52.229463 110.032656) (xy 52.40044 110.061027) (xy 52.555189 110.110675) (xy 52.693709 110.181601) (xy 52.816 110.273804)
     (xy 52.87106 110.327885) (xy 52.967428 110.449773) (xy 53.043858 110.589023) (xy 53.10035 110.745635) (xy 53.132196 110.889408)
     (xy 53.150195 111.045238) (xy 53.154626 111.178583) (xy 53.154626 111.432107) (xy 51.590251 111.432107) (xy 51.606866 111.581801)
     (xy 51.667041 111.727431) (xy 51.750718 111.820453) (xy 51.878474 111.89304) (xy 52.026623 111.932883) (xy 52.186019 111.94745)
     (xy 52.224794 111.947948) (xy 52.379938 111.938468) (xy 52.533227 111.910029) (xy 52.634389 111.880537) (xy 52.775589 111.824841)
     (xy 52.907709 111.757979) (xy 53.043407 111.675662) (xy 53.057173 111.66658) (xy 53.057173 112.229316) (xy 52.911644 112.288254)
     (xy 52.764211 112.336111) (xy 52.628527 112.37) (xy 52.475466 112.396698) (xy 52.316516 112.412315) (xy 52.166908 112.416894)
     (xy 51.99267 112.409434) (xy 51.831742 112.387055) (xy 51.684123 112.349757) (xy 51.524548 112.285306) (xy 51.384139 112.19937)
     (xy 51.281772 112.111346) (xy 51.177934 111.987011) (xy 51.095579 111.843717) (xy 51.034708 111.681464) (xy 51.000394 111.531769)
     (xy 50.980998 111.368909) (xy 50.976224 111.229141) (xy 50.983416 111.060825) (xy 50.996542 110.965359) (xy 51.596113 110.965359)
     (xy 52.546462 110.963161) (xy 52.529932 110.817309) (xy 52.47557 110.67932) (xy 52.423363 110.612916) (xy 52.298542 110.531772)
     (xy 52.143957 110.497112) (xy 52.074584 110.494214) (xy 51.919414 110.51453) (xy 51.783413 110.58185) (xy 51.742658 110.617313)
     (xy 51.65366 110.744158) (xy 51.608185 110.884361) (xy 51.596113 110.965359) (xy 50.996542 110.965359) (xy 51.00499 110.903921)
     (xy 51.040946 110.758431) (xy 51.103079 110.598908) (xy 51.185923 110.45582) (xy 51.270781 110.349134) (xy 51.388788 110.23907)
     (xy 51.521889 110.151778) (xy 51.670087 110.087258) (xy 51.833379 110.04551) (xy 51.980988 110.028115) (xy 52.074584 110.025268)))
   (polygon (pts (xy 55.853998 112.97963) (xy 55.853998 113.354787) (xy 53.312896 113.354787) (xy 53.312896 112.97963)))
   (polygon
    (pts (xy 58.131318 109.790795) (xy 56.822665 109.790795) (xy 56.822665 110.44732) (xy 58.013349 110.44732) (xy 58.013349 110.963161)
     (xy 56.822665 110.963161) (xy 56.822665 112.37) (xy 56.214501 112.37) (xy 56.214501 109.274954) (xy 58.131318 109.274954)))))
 (segment (start 48.26 86.995) (end 58.42 86.995) (width 0.2) (layer "F.Cu") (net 5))
 (segment (start 48.26 69.215) (end 48.26 86.995) (width 0.2) (layer "F.Cu") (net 5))
 (via (at 58.42 86.995) (size 1.6) (drill 1) (layers "F.Cu" "B.Cu") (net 5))
 (via (at 48.26 86.995) (size 1.6) (drill 1) (layers "F.Cu" "B.Cu") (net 5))
 (via (at 48.26 69.215) (size 1.6) (drill 1) (layers "F.Cu" "B.Cu") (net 5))
 (segment (start 58.42 104.775) (end 48.26 104.775) (width 1) (layer "B.Cu") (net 5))
 (segment (start 45.72 84.455) (end 45.72 86.995) (width 1) (layer "B.Cu") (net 5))
 (segment (start 40.64 56.515) (end 40.64 59.055) (width 1) (layer "B.Cu") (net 5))
 (segment (start 58.42 56.515) (end 58.42 59.055) (width 1) (layer "B.Cu") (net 5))
 (segment (start 40.64 79.375) (end 40.64 81.915) (width 1) (layer "B.Cu") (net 5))
 (segment (start 48.26 59.055) (end 58.42 59.055) (width 1) (layer "B.Cu") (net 5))
 (segment (start 40.64 104.775) (end 40.64 102.235) (width 1) (layer "B.Cu") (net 5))
 (segment (start 38.1 81.915) (end 38.1 97.155) (width 1) (layer "B.Cu") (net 5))
 (segment (start 38.1 104.775) (end 38.1 97.155) (width 1) (layer "B.Cu") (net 5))
 (segment (start 38.1 59.055) (end 38.1 71.755) (width 1) (layer "B.Cu") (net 5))
 (segment (start 45.72 86.995) (end 48.26 86.995) (width 1) (layer "B.Cu") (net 5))
 (segment (start 40.64 81.915) (end 38.1 81.915) (width 1) (layer "B.Cu") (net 5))
 (segment (start 58.42 102.235) (end 58.42 104.775) (width 1) (layer "B.Cu") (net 5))
 (segment (start 58.42 81.915) (end 58.42 86.995) (width 1) (layer "B.Cu") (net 5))
 (segment (start 48.26 66.675) (end 48.26 59.055) (width 1) (layer "B.Cu") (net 5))
 (segment (start 35.56 97.155) (end 38.1 97.155) (width 1) (layer "B.Cu") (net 5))
 (segment (start 48.26 104.775) (end 40.64 104.775) (width 1) (layer "B.Cu") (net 5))
 (segment (start 38.1 59.055) (end 38.1 51.435) (width 1) (layer "B.Cu") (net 5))
 (segment (start 58.42 79.375) (end 58.42 81.915) (width 1) (layer "B.Cu") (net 5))
 (segment (start 48.26 86.995) (end 48.26 104.775) (width 1) (layer "B.Cu") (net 5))
 (segment (start 40.64 59.055) (end 38.1 59.055) (width 1) (layer "B.Cu") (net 5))
 (segment (start 38.1 71.755) (end 38.1 81.915) (width 1) (layer "B.Cu") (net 5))
 (segment (start 35.56 71.755) (end 38.1 71.755) (width 1) (layer "B.Cu") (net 5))
 (segment (start 48.26 66.675) (end 48.26 69.215) (width 1) (layer "B.Cu") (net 5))
 (segment (start 40.64 104.775) (end 38.1 104.775) (width 1) (layer "B.Cu") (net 5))
 (segment (start 43.18 61.595) (end 43.18 48.895) (width 0.2) (layer "F.Cu") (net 4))
 (segment (start 38.1 94.615) (end 38.1 61.595) (width 0.2) (layer "F.Cu") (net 4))
 (segment (start 35.56 94.615) (end 38.1 94.615) (width 0.2) (layer "F.Cu") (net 4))
 (segment (start 43.18 48.895) (end 53.34 48.895) (width 0.2) (layer "F.Cu") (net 4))
 (segment (start 53.26 48.975) (end 53.34 48.895) (width 0.2) (layer "F.Cu") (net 4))
 (segment (start 53.26 61.595) (end 53.26 48.975) (width 0.2) (layer "F.Cu") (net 4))
 (segment (start 38.1 61.595) (end 43.18 61.595) (width 0.2) (layer "F.Cu") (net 4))
 (via (at 53.26 61.595) (size 1.6) (drill 1) (layers "F.Cu" "B.Cu") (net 4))
 (via (at 53.34 48.895) (size 1.6) (drill 1) (layers "F.Cu" "B.Cu") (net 4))
 (segment (start 38.1 48.895) (end 38.1 46.355) (width 1) (layer "B.Cu") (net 4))
 (segment (start 53.34 46.355) (end 53.34 48.895) (width 1) (layer "B.Cu") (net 4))
 (segment (start 53.34 66.675) (end 53.34 69.215) (width 1) (layer "B.Cu") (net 4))
 (segment (start 38.1 46.355) (end 53.34 46.355) (width 1) (layer "B.Cu") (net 4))
 (segment (start 35.56 48.895) (end 38.1 48.895) (width 1) (layer "B.Cu") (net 4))
 (segment (start 53.26 66.675) (end 53.26 61.595) (width 1) (layer "B.Cu") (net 4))
 (segment (start 45.72 51.435) (end 45.72 69.215) (width 1) (layer "B.Cu") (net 2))
 (segment (start 40.64 51.435) (end 45.72 51.435) (width 1) (layer "B.Cu") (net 2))
 (segment (start 40.64 51.435) (end 40.64 48.895) (width 1) (layer "B.Cu") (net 2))
 (segment (start 50.8 74.295) (end 50.8 51.435) (width 0.2) (layer "F.Cu") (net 11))
 (via (at 50.8 74.295) (size 1.6) (drill 1) (layers "F.Cu" "B.Cu") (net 11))
 (via (at 50.8 51.435) (size 1.6) (drill 1) (layers "F.Cu" "B.Cu") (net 11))
 (segment (start 53.34 74.295) (end 50.8 74.295) (width 1) (layer "B.Cu") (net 11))
 (segment (start 58.42 51.435) (end 50.8 51.435) (width 1) (layer "B.Cu") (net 11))
 (segment (start 58.42 51.435) (end 58.42 48.895) (width 1) (layer "B.Cu") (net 11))
 (segment (start 40.64 74.295) (end 45.72 74.295) (width 1) (layer "B.Cu") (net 3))
 (segment (start 40.64 74.295) (end 40.64 71.755) (width 1) (layer "B.Cu") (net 3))
 (segment (start 55.88 79.375) (end 55.88 74.295) (width 1) (layer "B.Cu") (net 10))
 (segment (start 55.88 74.295) (end 58.42 74.295) (width 1) (layer "B.Cu") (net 10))
 (segment (start 53.34 79.375) (end 55.88 79.375) (width 1) (layer "B.Cu") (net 10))
 (segment (start 58.42 74.295) (end 58.42 71.755) (width 1) (layer "B.Cu") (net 10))
 (segment (start 43.18 94.615) (end 43.18 79.375) (width 1) (layer "B.Cu") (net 1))
 (segment (start 40.64 97.155) (end 40.64 94.615) (width 1) (layer "B.Cu") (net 1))
 (segment (start 40.64 94.615) (end 43.18 94.615) (width 1) (layer "B.Cu") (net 1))
 (segment (start 43.18 79.375) (end 45.72 79.375) (width 1) (layer "B.Cu") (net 1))
 (segment (start 58.42 94.615) (end 58.42 97.155) (width 1) (layer "B.Cu") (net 9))
 (segment (start 53.34 97.155) (end 58.42 97.155) (width 1) (layer "B.Cu") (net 9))
 (segment (start 53.34 84.455) (end 53.34 97.155) (width 1) (layer "B.Cu") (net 9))
 (segment (start 45.72 71.755) (end 53.34 71.755) (width 1) (layer "B.Cu") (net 6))
 (segment (start 45.72 81.915) (end 53.34 81.915) (width 1) (layer "B.Cu") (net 8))
 (segment (start 45.72 76.835) (end 53.34 76.835) (width 1) (layer "B.Cu") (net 7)))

